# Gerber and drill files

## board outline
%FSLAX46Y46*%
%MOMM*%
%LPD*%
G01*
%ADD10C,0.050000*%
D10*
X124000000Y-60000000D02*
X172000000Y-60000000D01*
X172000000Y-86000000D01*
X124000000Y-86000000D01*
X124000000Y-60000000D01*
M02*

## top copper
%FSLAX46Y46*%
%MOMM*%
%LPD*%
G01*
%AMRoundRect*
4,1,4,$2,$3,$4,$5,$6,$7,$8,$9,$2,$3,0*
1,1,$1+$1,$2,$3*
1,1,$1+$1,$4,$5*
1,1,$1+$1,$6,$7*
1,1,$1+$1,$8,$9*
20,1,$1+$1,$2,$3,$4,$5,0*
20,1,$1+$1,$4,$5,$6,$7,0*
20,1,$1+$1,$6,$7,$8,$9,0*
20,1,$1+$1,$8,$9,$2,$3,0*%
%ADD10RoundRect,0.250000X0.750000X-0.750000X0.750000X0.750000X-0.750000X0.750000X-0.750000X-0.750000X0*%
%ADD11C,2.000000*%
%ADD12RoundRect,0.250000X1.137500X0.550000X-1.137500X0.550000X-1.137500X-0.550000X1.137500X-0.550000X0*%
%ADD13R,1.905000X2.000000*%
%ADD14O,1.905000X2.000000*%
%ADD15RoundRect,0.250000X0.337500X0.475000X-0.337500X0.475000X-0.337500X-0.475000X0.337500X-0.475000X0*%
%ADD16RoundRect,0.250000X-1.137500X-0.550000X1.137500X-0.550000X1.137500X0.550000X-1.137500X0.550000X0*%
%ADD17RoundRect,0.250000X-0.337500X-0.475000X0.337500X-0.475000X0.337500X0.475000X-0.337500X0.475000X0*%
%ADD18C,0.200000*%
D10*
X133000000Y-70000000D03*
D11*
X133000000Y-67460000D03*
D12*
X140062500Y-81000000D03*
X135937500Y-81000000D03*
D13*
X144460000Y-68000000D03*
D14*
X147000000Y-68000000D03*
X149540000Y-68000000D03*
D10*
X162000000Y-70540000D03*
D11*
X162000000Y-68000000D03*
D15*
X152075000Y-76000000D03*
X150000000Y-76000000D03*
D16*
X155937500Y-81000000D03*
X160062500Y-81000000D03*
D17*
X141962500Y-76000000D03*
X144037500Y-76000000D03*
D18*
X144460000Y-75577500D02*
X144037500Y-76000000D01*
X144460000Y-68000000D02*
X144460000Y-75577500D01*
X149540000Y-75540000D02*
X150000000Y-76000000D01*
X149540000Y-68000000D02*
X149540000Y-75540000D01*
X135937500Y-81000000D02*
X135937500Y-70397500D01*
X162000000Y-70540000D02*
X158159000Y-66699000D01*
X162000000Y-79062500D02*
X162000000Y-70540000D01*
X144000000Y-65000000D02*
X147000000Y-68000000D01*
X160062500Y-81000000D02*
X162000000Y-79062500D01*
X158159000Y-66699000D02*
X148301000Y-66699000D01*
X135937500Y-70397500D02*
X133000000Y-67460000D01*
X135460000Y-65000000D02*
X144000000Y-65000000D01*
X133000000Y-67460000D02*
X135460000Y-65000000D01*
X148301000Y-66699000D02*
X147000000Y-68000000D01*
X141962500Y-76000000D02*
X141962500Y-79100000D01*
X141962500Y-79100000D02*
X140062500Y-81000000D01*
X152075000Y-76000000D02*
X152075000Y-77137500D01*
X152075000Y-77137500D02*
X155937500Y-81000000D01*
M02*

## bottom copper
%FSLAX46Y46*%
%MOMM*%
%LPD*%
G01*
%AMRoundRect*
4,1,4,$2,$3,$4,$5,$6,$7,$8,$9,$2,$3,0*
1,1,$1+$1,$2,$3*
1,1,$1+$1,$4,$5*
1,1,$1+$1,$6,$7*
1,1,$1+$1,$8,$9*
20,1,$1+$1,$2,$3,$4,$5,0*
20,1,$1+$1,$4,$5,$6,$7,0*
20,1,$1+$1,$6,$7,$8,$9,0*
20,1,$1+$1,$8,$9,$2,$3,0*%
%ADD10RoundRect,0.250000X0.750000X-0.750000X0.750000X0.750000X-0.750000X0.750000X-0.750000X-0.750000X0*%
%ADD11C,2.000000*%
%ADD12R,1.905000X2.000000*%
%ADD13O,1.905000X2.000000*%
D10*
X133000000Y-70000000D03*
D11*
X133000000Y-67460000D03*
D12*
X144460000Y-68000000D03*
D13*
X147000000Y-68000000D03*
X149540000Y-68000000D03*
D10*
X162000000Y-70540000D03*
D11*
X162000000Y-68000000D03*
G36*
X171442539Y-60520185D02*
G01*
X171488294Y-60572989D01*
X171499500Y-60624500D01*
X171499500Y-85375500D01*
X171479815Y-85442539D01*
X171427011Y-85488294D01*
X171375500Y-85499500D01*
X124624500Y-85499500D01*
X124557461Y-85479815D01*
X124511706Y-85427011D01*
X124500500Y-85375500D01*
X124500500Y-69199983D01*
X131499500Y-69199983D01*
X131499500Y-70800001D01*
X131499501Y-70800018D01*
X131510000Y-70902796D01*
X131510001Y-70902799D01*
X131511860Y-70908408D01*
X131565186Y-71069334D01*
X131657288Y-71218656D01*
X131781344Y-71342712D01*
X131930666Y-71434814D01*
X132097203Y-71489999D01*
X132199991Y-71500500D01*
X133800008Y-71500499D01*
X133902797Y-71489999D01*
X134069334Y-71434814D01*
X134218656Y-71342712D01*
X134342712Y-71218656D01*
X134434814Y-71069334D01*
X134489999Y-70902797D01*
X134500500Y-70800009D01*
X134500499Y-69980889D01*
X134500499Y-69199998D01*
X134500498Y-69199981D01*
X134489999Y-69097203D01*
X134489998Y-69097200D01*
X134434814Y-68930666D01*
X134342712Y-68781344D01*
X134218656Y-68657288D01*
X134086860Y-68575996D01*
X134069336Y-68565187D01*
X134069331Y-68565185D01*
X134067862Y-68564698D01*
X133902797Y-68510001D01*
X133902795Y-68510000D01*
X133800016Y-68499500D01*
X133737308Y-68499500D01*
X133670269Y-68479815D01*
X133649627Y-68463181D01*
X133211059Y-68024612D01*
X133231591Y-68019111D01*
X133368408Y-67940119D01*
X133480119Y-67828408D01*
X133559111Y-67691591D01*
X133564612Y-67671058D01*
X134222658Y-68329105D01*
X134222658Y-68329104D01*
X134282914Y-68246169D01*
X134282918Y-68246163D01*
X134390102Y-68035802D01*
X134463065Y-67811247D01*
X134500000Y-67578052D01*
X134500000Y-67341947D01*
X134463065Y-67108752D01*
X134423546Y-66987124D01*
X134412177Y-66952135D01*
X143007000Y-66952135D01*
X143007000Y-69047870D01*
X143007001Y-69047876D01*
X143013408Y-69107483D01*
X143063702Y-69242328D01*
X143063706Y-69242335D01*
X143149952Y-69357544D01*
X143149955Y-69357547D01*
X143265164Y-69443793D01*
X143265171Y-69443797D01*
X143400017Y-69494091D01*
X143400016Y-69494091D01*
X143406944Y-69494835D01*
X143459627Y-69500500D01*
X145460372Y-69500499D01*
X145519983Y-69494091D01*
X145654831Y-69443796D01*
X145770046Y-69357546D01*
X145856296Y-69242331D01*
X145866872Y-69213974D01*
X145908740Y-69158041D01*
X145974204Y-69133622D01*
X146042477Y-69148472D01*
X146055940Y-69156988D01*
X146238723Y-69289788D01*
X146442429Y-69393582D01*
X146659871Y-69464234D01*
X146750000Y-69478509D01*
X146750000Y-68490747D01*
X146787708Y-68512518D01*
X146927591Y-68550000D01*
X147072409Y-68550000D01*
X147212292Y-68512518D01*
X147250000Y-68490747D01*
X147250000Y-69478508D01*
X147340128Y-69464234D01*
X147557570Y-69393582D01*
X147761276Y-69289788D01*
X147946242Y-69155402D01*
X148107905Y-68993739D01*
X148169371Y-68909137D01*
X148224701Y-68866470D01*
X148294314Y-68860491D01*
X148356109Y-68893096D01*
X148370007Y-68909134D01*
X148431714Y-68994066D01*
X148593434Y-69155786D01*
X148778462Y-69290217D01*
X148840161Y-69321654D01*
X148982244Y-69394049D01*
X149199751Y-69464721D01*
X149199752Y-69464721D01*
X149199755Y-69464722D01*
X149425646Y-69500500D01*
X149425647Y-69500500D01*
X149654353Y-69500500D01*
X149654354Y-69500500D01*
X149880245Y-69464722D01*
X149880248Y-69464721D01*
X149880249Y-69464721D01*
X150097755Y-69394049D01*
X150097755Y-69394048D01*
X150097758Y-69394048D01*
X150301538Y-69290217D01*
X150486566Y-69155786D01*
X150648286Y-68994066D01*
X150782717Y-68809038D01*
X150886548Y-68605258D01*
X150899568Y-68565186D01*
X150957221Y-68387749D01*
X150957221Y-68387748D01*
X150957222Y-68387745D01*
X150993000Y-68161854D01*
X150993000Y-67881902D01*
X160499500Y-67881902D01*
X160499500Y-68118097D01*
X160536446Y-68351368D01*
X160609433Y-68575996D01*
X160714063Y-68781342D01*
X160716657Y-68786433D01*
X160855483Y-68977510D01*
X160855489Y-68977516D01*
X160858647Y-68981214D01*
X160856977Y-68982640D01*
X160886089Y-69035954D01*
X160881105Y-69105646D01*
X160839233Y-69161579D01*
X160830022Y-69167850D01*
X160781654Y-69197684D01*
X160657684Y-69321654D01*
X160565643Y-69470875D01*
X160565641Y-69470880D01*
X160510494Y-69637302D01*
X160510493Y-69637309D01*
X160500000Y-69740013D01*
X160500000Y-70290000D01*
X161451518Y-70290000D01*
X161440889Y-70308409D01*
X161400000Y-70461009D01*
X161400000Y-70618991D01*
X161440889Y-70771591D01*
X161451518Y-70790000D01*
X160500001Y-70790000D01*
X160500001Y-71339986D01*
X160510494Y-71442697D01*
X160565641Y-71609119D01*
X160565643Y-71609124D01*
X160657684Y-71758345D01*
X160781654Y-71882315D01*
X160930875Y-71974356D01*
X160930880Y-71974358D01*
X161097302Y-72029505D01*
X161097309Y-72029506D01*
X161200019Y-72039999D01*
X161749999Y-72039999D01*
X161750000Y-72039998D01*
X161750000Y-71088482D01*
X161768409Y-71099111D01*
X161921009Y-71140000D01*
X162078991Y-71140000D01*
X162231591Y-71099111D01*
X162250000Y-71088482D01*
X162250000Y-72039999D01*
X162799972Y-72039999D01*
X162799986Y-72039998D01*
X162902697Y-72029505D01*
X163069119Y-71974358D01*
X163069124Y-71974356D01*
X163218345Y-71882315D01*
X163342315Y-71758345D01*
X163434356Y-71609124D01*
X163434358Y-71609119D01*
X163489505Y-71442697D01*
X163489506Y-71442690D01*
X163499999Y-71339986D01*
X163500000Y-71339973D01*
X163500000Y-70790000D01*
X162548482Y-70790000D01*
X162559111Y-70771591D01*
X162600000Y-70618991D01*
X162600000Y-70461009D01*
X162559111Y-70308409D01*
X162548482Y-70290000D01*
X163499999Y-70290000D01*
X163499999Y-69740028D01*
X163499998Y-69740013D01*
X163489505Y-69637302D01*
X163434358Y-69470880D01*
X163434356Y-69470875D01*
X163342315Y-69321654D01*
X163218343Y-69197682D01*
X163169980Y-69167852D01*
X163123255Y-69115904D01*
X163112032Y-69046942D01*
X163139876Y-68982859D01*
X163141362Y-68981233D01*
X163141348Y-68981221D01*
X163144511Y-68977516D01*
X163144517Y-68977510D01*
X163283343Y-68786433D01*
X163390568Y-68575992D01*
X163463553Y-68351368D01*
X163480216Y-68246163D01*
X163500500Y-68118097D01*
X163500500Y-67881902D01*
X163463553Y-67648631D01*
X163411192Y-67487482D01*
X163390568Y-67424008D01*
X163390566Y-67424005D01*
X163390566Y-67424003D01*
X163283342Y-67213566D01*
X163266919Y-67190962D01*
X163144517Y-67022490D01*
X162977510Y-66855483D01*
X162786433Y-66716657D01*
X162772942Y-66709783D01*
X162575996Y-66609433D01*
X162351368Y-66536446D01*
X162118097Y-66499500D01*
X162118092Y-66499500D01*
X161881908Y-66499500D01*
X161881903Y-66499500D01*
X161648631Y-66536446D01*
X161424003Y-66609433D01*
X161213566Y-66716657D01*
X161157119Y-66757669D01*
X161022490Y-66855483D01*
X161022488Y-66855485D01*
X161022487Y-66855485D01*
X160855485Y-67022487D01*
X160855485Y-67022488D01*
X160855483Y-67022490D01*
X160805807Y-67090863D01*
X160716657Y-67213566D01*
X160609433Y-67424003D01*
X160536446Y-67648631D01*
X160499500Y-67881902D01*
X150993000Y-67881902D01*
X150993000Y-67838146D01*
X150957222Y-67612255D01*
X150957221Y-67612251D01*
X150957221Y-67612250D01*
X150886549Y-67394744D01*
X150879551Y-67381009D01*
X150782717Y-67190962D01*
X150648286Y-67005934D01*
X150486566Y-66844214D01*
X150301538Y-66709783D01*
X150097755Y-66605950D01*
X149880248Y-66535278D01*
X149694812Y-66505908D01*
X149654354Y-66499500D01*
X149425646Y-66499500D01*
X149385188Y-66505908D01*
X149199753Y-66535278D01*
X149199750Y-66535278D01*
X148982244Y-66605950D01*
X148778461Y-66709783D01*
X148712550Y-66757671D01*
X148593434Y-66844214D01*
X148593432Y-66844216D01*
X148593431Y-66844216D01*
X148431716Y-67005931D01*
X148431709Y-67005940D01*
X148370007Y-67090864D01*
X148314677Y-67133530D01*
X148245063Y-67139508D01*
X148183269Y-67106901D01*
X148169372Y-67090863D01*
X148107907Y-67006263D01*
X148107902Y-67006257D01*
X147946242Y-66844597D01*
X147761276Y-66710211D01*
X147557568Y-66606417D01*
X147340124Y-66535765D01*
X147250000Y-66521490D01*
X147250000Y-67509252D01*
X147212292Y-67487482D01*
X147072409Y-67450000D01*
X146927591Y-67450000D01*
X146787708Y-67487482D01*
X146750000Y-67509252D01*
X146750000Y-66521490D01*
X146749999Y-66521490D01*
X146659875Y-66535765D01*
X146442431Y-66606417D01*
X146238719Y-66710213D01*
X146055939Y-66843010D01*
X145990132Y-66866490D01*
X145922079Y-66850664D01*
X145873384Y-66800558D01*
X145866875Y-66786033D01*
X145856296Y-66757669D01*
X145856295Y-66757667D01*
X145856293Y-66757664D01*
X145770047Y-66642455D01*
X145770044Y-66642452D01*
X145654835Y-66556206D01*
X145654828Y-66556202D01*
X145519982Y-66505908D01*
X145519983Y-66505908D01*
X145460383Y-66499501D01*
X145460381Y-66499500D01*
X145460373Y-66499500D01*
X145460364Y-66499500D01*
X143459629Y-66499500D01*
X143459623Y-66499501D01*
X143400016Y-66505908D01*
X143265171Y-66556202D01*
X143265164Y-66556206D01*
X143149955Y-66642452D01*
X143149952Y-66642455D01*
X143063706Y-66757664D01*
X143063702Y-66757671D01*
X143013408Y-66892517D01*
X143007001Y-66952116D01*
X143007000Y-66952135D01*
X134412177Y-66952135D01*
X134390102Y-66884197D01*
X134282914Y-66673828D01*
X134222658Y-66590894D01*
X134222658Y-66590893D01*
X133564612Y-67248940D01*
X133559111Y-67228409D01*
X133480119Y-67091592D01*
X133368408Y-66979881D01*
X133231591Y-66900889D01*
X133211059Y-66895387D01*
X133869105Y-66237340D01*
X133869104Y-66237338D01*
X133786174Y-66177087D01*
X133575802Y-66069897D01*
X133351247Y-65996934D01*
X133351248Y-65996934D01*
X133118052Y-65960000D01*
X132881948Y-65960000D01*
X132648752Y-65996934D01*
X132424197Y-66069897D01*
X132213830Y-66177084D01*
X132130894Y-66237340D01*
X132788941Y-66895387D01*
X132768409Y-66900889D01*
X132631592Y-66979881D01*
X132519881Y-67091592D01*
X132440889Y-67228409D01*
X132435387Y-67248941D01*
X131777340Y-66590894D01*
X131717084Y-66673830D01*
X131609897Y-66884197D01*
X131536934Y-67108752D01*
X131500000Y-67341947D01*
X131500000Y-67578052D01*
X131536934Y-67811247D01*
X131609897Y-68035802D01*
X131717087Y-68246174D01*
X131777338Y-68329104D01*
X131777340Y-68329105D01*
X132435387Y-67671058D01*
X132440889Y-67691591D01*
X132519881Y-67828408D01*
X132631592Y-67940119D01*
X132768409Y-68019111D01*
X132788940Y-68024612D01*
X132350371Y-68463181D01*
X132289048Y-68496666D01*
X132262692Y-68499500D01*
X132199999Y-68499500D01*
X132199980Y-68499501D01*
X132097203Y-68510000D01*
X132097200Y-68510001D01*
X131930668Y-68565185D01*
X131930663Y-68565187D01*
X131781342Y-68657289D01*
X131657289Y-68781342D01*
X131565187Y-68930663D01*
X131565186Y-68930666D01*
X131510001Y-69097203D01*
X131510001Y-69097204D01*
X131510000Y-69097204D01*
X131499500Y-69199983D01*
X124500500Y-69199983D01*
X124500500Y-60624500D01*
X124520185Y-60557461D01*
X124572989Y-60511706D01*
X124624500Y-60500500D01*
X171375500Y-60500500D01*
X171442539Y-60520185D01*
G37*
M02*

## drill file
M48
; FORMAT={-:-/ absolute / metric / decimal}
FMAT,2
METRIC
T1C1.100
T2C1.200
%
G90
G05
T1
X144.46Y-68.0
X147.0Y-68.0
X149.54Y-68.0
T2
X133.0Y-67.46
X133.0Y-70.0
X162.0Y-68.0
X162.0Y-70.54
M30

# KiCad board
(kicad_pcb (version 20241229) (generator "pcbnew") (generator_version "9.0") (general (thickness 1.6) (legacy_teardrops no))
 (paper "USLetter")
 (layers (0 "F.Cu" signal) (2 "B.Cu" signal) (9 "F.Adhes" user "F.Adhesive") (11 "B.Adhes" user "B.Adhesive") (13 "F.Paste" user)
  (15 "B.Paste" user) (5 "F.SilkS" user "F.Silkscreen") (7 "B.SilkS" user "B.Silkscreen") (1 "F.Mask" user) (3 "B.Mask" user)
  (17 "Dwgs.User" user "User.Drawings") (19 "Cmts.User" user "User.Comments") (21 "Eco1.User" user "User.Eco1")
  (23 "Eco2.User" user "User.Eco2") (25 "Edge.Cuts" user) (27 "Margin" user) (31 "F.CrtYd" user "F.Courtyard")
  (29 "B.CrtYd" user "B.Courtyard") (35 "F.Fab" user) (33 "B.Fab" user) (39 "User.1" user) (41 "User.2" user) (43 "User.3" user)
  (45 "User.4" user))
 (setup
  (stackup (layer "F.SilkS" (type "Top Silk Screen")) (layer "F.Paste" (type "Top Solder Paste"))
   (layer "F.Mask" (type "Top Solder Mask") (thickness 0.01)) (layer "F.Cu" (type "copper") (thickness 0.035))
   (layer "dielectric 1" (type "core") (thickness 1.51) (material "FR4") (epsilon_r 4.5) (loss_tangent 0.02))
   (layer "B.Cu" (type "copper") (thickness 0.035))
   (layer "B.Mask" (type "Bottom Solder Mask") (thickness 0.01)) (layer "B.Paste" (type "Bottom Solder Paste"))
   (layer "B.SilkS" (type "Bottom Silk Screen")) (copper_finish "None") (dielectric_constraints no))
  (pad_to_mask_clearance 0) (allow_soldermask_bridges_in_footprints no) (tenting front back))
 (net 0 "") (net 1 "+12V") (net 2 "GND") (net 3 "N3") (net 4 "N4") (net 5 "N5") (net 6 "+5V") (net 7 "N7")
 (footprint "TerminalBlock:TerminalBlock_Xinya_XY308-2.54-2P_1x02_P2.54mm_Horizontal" (layer "F.Cu") (at 133 70 90)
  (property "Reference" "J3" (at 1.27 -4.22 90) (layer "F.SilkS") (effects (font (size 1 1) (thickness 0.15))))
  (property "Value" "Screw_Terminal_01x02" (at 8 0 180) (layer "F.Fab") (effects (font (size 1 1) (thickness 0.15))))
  (pad "1" thru_hole roundrect (at 0 0 90) (size 2 2) (drill 1.2) (layers "*.Cu" "*.Mask") (remove_unused_layers no)
   (roundrect_rratio 0.125) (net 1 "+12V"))
  (pad "2" thru_hole circle (at 2.54 0 90) (size 2 2) (drill 1.2) (layers "*.Cu" "*.Mask") (remove_unused_layers no) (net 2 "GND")))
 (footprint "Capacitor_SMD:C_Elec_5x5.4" (layer "F.Cu") (at 138 81 180)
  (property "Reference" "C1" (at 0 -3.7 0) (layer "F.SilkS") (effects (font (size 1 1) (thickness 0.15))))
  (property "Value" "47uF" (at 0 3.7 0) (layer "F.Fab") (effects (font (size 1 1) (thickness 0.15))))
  (pad "1" smd roundrect (at -2.0625 0 180) (size 2.775 1.6) (layers "F.Cu" "F.Mask" "F.Paste") (roundrect_rratio 0.15625) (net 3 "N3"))
  (pad "2" smd roundrect (at 2.0625 0 180) (size 2.775 1.6) (layers "F.Cu" "F.Mask" "F.Paste") (roundrect_rratio 0.15625) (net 2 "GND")))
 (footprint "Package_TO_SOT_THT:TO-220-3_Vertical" (layer "F.Cu") (at 144.46 68)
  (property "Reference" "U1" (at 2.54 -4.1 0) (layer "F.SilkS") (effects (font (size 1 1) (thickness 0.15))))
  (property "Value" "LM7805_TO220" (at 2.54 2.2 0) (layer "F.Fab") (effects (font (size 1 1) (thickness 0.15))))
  (pad "1" thru_hole rect (at 0 0) (size 1.905 2) (drill 1.1) (layers "*.Cu" "*.Mask") (remove_unused_layers no) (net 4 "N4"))
  (pad "2" thru_hole oval (at 2.54 0) (size 1.905 2) (drill 1.1) (layers "*.Cu" "*.Mask") (remove_unused_layers no) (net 2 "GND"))
  (pad "3" thru_hole oval (at 5.08 0) (size 1.905 2) (drill 1.1) (layers "*.Cu" "*.Mask") (remove_unused_layers no) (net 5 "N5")))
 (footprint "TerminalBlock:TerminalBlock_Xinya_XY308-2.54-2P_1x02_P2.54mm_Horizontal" (layer "F.Cu") (at 162 70.54 90)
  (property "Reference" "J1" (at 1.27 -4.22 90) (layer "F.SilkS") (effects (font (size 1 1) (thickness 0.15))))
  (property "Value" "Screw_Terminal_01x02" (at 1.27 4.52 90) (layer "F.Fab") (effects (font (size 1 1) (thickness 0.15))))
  (pad "1" thru_hole roundrect (at 0 0 90) (size 2 2) (drill 1.2) (layers "*.Cu" "*.Mask") (remove_unused_layers no)
   (roundrect_rratio 0.125) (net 2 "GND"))
  (pad "2" thru_hole circle (at 2.54 0 90) (size 2 2) (drill 1.2) (layers "*.Cu" "*.Mask") (remove_unused_layers no) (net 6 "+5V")))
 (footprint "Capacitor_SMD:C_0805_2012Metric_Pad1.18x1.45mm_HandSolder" (layer "F.Cu") (at 151.0375 76 180)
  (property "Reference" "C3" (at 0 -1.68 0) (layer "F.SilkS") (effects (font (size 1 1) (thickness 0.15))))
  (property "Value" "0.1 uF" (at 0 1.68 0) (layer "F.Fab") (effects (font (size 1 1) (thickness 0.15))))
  (pad "1" smd roundrect (at -1.0375 0 180) (size 1.175 1.45) (layers "F.Cu" "F.Mask" "F.Paste") (roundrect_rratio 0.212766) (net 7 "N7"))
  (pad "2" smd roundrect (at 1.0375 0 180) (size 1.175 1.45) (layers "F.Cu" "F.Mask" "F.Paste") (roundrect_rratio 0.212766) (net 5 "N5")))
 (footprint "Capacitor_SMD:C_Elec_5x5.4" (layer "F.Cu") (at 158 81)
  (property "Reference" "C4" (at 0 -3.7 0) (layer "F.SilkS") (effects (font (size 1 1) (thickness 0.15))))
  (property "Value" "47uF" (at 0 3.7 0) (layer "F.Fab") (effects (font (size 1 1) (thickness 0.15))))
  (pad "1" smd roundrect (at -2.0625 0) (size 2.775 1.6) (layers "F.Cu" "F.Mask" "F.Paste") (roundrect_rratio 0.15625) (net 7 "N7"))
  (pad "2" smd roundrect (at 2.0625 0) (size 2.775 1.6) (layers "F.Cu" "F.Mask" "F.Paste") (roundrect_rratio 0.15625) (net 2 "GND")))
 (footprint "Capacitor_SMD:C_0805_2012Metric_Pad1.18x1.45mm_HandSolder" (layer "F.Cu") (at 143 76)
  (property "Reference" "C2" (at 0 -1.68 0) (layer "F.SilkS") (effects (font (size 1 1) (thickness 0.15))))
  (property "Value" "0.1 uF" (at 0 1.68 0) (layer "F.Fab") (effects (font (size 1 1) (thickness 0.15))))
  (pad "1" smd roundrect (at -1.0375 0) (size 1.175 1.45) (layers "F.Cu" "F.Mask" "F.Paste") (roundrect_rratio 0.212766) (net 3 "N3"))
  (pad "2" smd roundrect (at 1.0375 0) (size 1.175 1.45) (layers "F.Cu" "F.Mask" "F.Paste") (roundrect_rratio 0.212766) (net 4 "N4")))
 (gr_rect (start 124 60) (end 172 86) (stroke (width 0.05) (type default)) (fill no) (layer "Edge.Cuts"))
 (segment (start 144.46 75.5775) (end 144.0375 76) (width 0.2) (layer "F.Cu") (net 4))
 (segment (start 144.46 68) (end 144.46 75.5775) (width 0.2) (layer "F.Cu") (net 4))
 (segment (start 149.54 75.54) (end 150 76) (width 0.2) (layer "F.Cu") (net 5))
 (segment (start 149.54 68) (end 149.54 75.54) (width 0.2) (layer "F.Cu") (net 5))
 (segment (start 135.9375 81) (end 135.9375 70.3975) (width 0.2) (layer "F.Cu") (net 2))
 (segment (start 162 70.54) (end 158.159 66.699) (width 0.2) (layer "F.Cu") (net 2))
 (segment (start 162 79.0625) (end 162 70.54) (width 0.2) (layer "F.Cu") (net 2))
 (segment (start 144 65) (end 147 68) (width 0.2) (layer "F.Cu") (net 2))
 (segment (start 160.0625 81) (end 162 79.0625) (width 0.2) (layer "F.Cu") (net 2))
 (segment (start 158.159 66.699) (end 148.301 66.699) (width 0.2) (layer "F.Cu") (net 2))
 (segment (start 135.9375 70.3975) (end 133 67.46) (width 0.2) (layer "F.Cu") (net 2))
 (segment (start 135.46 65) (end 144 65) (width 0.2) (layer "F.Cu") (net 2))
 (segment (start 133 67.46) (end 135.46 65) (width 0.2) (layer "F.Cu") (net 2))
 (segment (start 148.301 66.699) (end 147 68) (width 0.2) (layer "F.Cu") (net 2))
 (segment (start 141.9625 76) (end 141.9625 79.1) (width 0.2) (layer "F.Cu") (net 3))
 (segment (start 141.9625 79.1) (end 140.0625 81) (width 0.2) (layer "F.Cu") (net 3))
 (segment (start 152.075 76) (end 152.075 77.1375) (width 0.2) (layer "F.Cu") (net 7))
 (segment (start 152.075 77.1375) (end 155.9375 81) (width 0.2) (layer "F.Cu") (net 7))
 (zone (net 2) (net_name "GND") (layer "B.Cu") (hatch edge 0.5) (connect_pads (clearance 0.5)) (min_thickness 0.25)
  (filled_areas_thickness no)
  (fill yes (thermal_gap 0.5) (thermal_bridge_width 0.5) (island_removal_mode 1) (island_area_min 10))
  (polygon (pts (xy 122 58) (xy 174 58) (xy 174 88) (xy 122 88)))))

